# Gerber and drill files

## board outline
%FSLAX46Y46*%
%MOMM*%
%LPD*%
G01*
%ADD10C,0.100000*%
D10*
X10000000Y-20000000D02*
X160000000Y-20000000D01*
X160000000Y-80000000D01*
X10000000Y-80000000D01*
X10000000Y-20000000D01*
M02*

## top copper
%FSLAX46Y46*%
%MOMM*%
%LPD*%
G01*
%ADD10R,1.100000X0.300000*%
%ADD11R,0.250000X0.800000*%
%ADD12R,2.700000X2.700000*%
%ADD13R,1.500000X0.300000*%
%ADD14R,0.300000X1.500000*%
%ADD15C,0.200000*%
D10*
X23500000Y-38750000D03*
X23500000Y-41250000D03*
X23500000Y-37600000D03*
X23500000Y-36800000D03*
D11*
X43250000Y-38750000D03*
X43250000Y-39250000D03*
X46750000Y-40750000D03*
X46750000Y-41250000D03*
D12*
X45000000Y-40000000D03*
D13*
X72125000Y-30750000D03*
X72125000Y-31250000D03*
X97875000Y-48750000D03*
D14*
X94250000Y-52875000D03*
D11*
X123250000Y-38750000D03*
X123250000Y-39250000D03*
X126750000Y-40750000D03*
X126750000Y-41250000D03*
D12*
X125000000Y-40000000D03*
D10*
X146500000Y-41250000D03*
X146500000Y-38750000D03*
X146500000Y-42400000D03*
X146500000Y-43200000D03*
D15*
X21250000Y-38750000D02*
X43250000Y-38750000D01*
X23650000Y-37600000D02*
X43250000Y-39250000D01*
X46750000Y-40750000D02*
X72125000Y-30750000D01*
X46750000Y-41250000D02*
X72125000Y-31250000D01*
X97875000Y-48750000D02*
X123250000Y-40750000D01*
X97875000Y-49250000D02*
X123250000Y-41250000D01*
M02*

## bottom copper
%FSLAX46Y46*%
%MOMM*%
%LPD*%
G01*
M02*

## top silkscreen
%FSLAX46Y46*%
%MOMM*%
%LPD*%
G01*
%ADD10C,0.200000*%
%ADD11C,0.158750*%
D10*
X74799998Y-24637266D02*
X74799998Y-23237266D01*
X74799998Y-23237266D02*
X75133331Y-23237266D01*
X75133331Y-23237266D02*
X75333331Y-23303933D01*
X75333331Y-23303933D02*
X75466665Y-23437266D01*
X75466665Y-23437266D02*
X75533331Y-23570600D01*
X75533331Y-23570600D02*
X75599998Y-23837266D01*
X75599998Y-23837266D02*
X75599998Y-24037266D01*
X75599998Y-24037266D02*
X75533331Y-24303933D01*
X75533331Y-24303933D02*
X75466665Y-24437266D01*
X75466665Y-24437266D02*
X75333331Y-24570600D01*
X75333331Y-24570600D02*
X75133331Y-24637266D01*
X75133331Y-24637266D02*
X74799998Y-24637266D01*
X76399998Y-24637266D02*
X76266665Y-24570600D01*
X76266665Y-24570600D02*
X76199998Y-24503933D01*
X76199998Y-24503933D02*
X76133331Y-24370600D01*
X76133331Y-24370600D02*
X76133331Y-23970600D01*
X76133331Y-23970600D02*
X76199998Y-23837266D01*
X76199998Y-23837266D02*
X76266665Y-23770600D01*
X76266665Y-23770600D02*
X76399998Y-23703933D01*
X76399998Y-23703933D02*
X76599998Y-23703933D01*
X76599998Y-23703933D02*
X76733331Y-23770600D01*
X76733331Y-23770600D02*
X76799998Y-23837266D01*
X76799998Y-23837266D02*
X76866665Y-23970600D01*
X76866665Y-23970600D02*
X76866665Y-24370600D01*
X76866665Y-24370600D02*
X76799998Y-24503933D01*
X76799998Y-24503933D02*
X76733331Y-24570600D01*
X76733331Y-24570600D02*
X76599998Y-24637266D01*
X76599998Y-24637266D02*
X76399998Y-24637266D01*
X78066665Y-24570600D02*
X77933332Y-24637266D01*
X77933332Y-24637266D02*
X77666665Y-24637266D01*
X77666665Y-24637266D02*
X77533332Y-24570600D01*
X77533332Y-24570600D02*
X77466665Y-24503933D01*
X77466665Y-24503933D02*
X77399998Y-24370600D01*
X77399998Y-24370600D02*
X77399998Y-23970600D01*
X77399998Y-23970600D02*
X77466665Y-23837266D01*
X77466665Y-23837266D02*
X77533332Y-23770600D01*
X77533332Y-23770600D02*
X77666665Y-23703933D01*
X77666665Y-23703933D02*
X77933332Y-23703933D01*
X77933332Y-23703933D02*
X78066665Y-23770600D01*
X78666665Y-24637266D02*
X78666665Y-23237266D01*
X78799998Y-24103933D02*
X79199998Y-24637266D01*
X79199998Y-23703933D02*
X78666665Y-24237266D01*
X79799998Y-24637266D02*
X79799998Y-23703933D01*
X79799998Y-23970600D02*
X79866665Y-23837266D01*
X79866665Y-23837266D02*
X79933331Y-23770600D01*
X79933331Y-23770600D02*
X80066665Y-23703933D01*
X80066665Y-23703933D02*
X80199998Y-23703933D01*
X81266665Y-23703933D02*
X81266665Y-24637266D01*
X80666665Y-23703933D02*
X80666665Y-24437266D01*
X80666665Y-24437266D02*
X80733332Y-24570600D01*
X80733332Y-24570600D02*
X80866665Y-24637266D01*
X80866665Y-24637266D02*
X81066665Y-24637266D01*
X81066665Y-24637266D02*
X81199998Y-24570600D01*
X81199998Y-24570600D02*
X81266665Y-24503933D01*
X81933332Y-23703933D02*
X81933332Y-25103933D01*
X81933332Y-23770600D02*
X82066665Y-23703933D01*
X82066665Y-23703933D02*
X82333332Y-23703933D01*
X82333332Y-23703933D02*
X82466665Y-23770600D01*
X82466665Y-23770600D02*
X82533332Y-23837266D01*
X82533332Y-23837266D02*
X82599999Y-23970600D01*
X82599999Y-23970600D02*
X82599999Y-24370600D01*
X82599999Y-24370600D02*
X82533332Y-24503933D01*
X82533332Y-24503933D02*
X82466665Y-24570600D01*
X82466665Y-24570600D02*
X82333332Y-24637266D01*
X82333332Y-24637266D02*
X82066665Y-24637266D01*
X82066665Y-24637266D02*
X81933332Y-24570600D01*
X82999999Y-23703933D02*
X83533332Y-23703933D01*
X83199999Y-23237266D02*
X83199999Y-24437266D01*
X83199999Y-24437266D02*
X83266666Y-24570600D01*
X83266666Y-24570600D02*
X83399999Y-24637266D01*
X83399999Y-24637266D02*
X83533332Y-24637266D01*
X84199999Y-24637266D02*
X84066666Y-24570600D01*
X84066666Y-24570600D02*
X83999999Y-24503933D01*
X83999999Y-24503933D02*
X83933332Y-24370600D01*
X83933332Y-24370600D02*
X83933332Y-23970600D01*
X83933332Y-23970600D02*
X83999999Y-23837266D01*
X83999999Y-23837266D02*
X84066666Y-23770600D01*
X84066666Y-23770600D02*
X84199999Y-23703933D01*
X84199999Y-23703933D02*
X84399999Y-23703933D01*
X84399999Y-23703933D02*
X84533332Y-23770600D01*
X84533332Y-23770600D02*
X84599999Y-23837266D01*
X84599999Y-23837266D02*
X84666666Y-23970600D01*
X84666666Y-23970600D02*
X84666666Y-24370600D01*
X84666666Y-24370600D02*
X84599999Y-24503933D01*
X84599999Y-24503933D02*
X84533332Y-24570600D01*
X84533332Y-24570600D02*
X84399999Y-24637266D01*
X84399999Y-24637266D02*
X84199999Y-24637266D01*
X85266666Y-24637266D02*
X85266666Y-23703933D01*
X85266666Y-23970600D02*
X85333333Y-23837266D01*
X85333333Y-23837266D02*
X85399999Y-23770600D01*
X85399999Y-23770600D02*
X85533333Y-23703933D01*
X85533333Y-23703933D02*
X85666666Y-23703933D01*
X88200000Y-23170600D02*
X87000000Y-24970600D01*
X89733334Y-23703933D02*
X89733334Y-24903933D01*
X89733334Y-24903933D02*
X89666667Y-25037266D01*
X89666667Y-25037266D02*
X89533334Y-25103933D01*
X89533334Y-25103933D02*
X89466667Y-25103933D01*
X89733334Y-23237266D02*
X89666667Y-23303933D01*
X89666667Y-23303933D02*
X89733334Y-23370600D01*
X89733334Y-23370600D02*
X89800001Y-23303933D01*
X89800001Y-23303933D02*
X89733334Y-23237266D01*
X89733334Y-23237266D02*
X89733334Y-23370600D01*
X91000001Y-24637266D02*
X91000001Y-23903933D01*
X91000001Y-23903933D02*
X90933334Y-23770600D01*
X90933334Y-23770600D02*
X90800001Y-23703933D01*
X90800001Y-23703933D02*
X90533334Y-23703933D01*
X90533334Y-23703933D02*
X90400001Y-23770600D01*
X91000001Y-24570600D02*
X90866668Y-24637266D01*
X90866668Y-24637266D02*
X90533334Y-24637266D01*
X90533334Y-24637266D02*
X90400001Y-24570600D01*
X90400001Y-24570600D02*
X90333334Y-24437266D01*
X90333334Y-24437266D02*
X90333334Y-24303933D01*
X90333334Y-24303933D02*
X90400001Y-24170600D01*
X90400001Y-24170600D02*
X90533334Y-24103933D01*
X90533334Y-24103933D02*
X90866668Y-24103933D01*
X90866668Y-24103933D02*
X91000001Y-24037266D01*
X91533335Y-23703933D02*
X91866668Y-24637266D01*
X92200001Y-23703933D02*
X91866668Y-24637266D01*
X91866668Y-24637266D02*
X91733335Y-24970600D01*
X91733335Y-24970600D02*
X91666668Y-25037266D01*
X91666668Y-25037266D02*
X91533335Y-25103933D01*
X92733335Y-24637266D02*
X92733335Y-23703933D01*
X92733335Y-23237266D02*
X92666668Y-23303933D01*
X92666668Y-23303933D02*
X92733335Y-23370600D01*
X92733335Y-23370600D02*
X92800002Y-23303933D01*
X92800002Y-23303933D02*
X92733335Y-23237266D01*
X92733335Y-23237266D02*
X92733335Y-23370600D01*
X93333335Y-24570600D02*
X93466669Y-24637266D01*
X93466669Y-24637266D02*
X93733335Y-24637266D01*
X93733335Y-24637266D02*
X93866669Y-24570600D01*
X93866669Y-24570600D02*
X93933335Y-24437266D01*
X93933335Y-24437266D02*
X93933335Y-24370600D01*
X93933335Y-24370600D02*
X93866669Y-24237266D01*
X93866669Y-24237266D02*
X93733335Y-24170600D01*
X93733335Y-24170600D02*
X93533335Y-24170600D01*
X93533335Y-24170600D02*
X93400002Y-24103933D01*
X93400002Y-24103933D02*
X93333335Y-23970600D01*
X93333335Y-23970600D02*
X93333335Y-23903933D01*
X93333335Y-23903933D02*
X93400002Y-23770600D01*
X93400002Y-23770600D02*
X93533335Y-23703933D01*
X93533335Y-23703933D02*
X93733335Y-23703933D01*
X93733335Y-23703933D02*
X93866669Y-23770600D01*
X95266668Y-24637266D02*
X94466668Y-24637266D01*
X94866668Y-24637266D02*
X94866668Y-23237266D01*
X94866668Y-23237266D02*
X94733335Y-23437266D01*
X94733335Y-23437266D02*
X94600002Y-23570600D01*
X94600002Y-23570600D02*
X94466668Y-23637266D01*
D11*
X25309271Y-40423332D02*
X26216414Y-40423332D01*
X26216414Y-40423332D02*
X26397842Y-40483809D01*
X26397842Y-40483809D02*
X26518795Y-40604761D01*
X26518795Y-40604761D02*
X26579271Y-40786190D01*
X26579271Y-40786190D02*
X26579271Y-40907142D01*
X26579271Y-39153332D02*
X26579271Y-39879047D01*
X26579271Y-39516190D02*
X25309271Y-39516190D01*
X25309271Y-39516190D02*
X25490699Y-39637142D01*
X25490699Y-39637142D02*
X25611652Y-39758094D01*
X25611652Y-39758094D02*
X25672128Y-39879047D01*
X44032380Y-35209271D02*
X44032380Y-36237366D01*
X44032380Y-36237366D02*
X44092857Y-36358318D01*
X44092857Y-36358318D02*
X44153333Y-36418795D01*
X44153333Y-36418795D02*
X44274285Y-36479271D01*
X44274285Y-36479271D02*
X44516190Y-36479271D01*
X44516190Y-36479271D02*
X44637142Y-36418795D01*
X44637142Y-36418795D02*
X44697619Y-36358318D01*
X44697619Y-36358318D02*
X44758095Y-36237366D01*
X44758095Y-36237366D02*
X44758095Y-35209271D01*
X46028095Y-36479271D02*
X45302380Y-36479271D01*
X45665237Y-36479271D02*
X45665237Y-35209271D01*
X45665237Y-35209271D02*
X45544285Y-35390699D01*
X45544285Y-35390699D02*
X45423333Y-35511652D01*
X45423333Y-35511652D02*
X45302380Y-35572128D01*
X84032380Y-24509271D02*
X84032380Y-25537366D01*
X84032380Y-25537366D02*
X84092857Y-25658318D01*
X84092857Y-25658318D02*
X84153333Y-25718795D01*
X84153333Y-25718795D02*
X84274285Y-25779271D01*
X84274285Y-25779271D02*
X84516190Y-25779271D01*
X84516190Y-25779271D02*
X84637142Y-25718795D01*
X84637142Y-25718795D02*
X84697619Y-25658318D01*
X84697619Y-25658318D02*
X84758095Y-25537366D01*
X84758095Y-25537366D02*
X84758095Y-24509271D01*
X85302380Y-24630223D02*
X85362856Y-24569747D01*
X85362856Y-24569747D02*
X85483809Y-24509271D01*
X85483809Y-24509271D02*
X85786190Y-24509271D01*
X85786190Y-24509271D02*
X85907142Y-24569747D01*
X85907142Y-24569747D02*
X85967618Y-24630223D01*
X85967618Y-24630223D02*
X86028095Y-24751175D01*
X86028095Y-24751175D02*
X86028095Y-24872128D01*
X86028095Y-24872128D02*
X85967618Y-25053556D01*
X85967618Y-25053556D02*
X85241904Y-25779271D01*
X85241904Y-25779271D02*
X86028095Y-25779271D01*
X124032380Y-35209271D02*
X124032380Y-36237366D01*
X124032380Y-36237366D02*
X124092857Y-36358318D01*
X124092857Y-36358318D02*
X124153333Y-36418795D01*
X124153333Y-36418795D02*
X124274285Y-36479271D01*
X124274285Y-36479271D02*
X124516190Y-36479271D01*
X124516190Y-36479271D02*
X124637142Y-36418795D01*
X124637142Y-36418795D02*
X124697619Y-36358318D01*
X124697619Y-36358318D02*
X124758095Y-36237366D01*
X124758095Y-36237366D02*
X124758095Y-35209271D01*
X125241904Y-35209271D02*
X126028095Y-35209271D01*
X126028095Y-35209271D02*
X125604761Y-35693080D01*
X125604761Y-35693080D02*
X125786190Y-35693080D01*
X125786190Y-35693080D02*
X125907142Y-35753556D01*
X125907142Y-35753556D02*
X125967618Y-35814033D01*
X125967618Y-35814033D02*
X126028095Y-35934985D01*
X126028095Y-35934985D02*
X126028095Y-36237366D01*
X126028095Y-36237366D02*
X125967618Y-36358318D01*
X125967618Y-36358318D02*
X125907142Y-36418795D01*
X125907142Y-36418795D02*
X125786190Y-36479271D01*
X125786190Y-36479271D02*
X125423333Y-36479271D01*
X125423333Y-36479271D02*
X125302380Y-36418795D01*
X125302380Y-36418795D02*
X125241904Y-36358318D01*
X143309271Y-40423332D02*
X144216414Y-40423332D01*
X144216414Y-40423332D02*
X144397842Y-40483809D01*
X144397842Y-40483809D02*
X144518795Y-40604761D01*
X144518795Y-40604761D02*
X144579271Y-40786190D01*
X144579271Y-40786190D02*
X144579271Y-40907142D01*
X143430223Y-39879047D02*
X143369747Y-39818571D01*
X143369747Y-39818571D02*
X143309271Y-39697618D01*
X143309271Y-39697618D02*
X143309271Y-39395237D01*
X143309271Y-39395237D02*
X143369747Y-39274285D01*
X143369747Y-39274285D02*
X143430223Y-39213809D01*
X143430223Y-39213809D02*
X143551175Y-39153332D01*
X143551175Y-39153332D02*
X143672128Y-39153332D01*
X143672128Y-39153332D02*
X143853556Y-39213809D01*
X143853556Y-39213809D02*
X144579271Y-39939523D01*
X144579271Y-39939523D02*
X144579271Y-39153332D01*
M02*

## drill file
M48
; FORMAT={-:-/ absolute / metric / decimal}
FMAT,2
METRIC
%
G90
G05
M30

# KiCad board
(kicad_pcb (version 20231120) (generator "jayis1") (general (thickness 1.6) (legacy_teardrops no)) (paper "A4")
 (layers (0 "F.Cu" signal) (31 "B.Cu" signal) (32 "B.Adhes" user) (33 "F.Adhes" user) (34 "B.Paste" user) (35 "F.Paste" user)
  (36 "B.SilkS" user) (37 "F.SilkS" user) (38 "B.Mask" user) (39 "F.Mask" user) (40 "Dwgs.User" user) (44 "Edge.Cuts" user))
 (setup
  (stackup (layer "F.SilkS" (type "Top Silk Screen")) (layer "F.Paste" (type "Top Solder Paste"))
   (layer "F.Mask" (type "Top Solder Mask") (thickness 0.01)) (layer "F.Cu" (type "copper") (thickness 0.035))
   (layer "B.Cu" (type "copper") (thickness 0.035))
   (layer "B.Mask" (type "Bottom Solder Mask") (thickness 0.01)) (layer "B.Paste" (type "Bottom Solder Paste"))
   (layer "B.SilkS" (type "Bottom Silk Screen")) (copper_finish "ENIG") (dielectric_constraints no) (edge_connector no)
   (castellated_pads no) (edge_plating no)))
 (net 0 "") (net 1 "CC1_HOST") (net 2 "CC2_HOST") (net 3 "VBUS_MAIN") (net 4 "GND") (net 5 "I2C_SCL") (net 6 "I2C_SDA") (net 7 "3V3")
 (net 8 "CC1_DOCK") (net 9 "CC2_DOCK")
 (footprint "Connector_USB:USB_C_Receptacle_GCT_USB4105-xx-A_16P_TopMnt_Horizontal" (layer "F.Cu") (at 20 40 270)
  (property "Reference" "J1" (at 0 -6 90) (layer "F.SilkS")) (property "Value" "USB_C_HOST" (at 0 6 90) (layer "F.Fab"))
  (pad "A5" smd rect (at -1.25 -3.5 270) (size 0.3 1.1) (layers "F.Cu" "F.Paste" "F.Mask") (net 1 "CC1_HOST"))
  (pad "B5" smd rect (at 1.25 -3.5 270) (size 0.3 1.1) (layers "F.Cu" "F.Paste" "F.Mask") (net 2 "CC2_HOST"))
  (pad "A4" smd rect (at -2.4 -3.5 270) (size 0.3 1.1) (layers "F.Cu" "F.Paste" "F.Mask") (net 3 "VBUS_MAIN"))
  (pad "A1" smd rect (at -3.2 -3.5 270) (size 0.3 1.1) (layers "F.Cu" "F.Paste" "F.Mask") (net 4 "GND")))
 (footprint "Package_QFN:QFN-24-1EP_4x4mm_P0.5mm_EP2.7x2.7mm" (layer "F.Cu") (at 45 40)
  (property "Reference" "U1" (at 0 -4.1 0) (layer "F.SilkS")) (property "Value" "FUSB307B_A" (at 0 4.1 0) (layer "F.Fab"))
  (pad "1" smd rect (at -1.75 -1.25) (size 0.25 0.8) (layers "F.Cu" "F.Paste" "F.Mask") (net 1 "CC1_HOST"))
  (pad "2" smd rect (at -1.75 -0.75) (size 0.25 0.8) (layers "F.Cu" "F.Paste" "F.Mask") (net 2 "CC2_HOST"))
  (pad "23" smd rect (at 1.75 0.75) (size 0.25 0.8) (layers "F.Cu" "F.Paste" "F.Mask") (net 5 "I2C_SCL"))
  (pad "24" smd rect (at 1.75 1.25) (size 0.25 0.8) (layers "F.Cu" "F.Paste" "F.Mask") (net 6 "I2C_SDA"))
  (pad "25" smd rect (at 0 0) (size 2.7 2.7) (layers "F.Cu" "F.Mask") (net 4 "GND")))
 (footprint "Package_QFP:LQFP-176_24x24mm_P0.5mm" (layer "F.Cu") (at 85 40) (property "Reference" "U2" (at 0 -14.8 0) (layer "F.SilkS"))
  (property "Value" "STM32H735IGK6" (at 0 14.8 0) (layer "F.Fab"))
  (pad "12" smd rect (at -12.875 -9.25) (size 1.5 0.3) (layers "F.Cu" "F.Paste" "F.Mask") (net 5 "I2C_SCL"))
  (pad "13" smd rect (at -12.875 -8.75) (size 1.5 0.3) (layers "F.Cu" "F.Paste" "F.Mask") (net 6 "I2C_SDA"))
  (pad "68" smd rect (at 12.875 8.75) (size 1.5 0.3) (layers "F.Cu" "F.Paste" "F.Mask") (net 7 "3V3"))
  (pad "89" smd rect (at 9.25 12.875 90) (size 1.5 0.3) (layers "F.Cu" "F.Paste" "F.Mask") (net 4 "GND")))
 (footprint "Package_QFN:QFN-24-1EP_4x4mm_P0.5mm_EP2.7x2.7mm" (layer "F.Cu") (at 125 40)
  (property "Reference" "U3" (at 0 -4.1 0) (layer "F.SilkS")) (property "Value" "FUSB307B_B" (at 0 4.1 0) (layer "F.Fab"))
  (pad "1" smd rect (at -1.75 -1.25) (size 0.25 0.8) (layers "F.Cu" "F.Paste" "F.Mask") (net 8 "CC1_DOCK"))
  (pad "2" smd rect (at -1.75 -0.75) (size 0.25 0.8) (layers "F.Cu" "F.Paste" "F.Mask") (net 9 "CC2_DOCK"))
  (pad "23" smd rect (at 1.75 0.75) (size 0.25 0.8) (layers "F.Cu" "F.Paste" "F.Mask") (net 5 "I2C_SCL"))
  (pad "24" smd rect (at 1.75 1.25) (size 0.25 0.8) (layers "F.Cu" "F.Paste" "F.Mask") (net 6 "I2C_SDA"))
  (pad "25" smd rect (at 0 0) (size 2.7 2.7) (layers "F.Cu" "F.Mask") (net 4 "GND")))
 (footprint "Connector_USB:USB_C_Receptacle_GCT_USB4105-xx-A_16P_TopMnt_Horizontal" (layer "F.Cu") (at 150 40 90)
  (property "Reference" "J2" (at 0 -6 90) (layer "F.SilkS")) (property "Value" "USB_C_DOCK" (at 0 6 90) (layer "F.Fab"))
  (pad "A5" smd rect (at -1.25 -3.5 90) (size 0.3 1.1) (layers "F.Cu" "F.Paste" "F.Mask") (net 8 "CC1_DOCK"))
  (pad "B5" smd rect (at 1.25 -3.5 90) (size 0.3 1.1) (layers "F.Cu" "F.Paste" "F.Mask") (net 9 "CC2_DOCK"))
  (pad "A4" smd rect (at -2.4 -3.5 90) (size 0.3 1.1) (layers "F.Cu" "F.Paste" "F.Mask") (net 3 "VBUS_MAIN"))
  (pad "A1" smd rect (at -3.2 -3.5 90) (size 0.3 1.1) (layers "F.Cu" "F.Paste" "F.Mask") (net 4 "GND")))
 (segment (start 21.25 38.75) (end 43.25 38.75) (width 0.2) (layer "F.Cu") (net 1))
 (segment (start 23.65 37.6) (end 43.25 39.25) (width 0.2) (layer "F.Cu") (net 2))
 (segment (start 46.75 40.75) (end 72.125 30.75) (width 0.2) (layer "F.Cu") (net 5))
 (segment (start 46.75 41.25) (end 72.125 31.25) (width 0.2) (layer "F.Cu") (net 6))
 (segment (start 97.875 48.75) (end 123.25 40.75) (width 0.2) (layer "F.Cu") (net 5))
 (segment (start 97.875 49.25) (end 123.25 41.25) (width 0.2) (layer "F.Cu") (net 6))
 (gr_rect (start 10 20) (end 160 80) (stroke (width 0.1) (type default)) (fill no) (layer "Edge.Cuts"))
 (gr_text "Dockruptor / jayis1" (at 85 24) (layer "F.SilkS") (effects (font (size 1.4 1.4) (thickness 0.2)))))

